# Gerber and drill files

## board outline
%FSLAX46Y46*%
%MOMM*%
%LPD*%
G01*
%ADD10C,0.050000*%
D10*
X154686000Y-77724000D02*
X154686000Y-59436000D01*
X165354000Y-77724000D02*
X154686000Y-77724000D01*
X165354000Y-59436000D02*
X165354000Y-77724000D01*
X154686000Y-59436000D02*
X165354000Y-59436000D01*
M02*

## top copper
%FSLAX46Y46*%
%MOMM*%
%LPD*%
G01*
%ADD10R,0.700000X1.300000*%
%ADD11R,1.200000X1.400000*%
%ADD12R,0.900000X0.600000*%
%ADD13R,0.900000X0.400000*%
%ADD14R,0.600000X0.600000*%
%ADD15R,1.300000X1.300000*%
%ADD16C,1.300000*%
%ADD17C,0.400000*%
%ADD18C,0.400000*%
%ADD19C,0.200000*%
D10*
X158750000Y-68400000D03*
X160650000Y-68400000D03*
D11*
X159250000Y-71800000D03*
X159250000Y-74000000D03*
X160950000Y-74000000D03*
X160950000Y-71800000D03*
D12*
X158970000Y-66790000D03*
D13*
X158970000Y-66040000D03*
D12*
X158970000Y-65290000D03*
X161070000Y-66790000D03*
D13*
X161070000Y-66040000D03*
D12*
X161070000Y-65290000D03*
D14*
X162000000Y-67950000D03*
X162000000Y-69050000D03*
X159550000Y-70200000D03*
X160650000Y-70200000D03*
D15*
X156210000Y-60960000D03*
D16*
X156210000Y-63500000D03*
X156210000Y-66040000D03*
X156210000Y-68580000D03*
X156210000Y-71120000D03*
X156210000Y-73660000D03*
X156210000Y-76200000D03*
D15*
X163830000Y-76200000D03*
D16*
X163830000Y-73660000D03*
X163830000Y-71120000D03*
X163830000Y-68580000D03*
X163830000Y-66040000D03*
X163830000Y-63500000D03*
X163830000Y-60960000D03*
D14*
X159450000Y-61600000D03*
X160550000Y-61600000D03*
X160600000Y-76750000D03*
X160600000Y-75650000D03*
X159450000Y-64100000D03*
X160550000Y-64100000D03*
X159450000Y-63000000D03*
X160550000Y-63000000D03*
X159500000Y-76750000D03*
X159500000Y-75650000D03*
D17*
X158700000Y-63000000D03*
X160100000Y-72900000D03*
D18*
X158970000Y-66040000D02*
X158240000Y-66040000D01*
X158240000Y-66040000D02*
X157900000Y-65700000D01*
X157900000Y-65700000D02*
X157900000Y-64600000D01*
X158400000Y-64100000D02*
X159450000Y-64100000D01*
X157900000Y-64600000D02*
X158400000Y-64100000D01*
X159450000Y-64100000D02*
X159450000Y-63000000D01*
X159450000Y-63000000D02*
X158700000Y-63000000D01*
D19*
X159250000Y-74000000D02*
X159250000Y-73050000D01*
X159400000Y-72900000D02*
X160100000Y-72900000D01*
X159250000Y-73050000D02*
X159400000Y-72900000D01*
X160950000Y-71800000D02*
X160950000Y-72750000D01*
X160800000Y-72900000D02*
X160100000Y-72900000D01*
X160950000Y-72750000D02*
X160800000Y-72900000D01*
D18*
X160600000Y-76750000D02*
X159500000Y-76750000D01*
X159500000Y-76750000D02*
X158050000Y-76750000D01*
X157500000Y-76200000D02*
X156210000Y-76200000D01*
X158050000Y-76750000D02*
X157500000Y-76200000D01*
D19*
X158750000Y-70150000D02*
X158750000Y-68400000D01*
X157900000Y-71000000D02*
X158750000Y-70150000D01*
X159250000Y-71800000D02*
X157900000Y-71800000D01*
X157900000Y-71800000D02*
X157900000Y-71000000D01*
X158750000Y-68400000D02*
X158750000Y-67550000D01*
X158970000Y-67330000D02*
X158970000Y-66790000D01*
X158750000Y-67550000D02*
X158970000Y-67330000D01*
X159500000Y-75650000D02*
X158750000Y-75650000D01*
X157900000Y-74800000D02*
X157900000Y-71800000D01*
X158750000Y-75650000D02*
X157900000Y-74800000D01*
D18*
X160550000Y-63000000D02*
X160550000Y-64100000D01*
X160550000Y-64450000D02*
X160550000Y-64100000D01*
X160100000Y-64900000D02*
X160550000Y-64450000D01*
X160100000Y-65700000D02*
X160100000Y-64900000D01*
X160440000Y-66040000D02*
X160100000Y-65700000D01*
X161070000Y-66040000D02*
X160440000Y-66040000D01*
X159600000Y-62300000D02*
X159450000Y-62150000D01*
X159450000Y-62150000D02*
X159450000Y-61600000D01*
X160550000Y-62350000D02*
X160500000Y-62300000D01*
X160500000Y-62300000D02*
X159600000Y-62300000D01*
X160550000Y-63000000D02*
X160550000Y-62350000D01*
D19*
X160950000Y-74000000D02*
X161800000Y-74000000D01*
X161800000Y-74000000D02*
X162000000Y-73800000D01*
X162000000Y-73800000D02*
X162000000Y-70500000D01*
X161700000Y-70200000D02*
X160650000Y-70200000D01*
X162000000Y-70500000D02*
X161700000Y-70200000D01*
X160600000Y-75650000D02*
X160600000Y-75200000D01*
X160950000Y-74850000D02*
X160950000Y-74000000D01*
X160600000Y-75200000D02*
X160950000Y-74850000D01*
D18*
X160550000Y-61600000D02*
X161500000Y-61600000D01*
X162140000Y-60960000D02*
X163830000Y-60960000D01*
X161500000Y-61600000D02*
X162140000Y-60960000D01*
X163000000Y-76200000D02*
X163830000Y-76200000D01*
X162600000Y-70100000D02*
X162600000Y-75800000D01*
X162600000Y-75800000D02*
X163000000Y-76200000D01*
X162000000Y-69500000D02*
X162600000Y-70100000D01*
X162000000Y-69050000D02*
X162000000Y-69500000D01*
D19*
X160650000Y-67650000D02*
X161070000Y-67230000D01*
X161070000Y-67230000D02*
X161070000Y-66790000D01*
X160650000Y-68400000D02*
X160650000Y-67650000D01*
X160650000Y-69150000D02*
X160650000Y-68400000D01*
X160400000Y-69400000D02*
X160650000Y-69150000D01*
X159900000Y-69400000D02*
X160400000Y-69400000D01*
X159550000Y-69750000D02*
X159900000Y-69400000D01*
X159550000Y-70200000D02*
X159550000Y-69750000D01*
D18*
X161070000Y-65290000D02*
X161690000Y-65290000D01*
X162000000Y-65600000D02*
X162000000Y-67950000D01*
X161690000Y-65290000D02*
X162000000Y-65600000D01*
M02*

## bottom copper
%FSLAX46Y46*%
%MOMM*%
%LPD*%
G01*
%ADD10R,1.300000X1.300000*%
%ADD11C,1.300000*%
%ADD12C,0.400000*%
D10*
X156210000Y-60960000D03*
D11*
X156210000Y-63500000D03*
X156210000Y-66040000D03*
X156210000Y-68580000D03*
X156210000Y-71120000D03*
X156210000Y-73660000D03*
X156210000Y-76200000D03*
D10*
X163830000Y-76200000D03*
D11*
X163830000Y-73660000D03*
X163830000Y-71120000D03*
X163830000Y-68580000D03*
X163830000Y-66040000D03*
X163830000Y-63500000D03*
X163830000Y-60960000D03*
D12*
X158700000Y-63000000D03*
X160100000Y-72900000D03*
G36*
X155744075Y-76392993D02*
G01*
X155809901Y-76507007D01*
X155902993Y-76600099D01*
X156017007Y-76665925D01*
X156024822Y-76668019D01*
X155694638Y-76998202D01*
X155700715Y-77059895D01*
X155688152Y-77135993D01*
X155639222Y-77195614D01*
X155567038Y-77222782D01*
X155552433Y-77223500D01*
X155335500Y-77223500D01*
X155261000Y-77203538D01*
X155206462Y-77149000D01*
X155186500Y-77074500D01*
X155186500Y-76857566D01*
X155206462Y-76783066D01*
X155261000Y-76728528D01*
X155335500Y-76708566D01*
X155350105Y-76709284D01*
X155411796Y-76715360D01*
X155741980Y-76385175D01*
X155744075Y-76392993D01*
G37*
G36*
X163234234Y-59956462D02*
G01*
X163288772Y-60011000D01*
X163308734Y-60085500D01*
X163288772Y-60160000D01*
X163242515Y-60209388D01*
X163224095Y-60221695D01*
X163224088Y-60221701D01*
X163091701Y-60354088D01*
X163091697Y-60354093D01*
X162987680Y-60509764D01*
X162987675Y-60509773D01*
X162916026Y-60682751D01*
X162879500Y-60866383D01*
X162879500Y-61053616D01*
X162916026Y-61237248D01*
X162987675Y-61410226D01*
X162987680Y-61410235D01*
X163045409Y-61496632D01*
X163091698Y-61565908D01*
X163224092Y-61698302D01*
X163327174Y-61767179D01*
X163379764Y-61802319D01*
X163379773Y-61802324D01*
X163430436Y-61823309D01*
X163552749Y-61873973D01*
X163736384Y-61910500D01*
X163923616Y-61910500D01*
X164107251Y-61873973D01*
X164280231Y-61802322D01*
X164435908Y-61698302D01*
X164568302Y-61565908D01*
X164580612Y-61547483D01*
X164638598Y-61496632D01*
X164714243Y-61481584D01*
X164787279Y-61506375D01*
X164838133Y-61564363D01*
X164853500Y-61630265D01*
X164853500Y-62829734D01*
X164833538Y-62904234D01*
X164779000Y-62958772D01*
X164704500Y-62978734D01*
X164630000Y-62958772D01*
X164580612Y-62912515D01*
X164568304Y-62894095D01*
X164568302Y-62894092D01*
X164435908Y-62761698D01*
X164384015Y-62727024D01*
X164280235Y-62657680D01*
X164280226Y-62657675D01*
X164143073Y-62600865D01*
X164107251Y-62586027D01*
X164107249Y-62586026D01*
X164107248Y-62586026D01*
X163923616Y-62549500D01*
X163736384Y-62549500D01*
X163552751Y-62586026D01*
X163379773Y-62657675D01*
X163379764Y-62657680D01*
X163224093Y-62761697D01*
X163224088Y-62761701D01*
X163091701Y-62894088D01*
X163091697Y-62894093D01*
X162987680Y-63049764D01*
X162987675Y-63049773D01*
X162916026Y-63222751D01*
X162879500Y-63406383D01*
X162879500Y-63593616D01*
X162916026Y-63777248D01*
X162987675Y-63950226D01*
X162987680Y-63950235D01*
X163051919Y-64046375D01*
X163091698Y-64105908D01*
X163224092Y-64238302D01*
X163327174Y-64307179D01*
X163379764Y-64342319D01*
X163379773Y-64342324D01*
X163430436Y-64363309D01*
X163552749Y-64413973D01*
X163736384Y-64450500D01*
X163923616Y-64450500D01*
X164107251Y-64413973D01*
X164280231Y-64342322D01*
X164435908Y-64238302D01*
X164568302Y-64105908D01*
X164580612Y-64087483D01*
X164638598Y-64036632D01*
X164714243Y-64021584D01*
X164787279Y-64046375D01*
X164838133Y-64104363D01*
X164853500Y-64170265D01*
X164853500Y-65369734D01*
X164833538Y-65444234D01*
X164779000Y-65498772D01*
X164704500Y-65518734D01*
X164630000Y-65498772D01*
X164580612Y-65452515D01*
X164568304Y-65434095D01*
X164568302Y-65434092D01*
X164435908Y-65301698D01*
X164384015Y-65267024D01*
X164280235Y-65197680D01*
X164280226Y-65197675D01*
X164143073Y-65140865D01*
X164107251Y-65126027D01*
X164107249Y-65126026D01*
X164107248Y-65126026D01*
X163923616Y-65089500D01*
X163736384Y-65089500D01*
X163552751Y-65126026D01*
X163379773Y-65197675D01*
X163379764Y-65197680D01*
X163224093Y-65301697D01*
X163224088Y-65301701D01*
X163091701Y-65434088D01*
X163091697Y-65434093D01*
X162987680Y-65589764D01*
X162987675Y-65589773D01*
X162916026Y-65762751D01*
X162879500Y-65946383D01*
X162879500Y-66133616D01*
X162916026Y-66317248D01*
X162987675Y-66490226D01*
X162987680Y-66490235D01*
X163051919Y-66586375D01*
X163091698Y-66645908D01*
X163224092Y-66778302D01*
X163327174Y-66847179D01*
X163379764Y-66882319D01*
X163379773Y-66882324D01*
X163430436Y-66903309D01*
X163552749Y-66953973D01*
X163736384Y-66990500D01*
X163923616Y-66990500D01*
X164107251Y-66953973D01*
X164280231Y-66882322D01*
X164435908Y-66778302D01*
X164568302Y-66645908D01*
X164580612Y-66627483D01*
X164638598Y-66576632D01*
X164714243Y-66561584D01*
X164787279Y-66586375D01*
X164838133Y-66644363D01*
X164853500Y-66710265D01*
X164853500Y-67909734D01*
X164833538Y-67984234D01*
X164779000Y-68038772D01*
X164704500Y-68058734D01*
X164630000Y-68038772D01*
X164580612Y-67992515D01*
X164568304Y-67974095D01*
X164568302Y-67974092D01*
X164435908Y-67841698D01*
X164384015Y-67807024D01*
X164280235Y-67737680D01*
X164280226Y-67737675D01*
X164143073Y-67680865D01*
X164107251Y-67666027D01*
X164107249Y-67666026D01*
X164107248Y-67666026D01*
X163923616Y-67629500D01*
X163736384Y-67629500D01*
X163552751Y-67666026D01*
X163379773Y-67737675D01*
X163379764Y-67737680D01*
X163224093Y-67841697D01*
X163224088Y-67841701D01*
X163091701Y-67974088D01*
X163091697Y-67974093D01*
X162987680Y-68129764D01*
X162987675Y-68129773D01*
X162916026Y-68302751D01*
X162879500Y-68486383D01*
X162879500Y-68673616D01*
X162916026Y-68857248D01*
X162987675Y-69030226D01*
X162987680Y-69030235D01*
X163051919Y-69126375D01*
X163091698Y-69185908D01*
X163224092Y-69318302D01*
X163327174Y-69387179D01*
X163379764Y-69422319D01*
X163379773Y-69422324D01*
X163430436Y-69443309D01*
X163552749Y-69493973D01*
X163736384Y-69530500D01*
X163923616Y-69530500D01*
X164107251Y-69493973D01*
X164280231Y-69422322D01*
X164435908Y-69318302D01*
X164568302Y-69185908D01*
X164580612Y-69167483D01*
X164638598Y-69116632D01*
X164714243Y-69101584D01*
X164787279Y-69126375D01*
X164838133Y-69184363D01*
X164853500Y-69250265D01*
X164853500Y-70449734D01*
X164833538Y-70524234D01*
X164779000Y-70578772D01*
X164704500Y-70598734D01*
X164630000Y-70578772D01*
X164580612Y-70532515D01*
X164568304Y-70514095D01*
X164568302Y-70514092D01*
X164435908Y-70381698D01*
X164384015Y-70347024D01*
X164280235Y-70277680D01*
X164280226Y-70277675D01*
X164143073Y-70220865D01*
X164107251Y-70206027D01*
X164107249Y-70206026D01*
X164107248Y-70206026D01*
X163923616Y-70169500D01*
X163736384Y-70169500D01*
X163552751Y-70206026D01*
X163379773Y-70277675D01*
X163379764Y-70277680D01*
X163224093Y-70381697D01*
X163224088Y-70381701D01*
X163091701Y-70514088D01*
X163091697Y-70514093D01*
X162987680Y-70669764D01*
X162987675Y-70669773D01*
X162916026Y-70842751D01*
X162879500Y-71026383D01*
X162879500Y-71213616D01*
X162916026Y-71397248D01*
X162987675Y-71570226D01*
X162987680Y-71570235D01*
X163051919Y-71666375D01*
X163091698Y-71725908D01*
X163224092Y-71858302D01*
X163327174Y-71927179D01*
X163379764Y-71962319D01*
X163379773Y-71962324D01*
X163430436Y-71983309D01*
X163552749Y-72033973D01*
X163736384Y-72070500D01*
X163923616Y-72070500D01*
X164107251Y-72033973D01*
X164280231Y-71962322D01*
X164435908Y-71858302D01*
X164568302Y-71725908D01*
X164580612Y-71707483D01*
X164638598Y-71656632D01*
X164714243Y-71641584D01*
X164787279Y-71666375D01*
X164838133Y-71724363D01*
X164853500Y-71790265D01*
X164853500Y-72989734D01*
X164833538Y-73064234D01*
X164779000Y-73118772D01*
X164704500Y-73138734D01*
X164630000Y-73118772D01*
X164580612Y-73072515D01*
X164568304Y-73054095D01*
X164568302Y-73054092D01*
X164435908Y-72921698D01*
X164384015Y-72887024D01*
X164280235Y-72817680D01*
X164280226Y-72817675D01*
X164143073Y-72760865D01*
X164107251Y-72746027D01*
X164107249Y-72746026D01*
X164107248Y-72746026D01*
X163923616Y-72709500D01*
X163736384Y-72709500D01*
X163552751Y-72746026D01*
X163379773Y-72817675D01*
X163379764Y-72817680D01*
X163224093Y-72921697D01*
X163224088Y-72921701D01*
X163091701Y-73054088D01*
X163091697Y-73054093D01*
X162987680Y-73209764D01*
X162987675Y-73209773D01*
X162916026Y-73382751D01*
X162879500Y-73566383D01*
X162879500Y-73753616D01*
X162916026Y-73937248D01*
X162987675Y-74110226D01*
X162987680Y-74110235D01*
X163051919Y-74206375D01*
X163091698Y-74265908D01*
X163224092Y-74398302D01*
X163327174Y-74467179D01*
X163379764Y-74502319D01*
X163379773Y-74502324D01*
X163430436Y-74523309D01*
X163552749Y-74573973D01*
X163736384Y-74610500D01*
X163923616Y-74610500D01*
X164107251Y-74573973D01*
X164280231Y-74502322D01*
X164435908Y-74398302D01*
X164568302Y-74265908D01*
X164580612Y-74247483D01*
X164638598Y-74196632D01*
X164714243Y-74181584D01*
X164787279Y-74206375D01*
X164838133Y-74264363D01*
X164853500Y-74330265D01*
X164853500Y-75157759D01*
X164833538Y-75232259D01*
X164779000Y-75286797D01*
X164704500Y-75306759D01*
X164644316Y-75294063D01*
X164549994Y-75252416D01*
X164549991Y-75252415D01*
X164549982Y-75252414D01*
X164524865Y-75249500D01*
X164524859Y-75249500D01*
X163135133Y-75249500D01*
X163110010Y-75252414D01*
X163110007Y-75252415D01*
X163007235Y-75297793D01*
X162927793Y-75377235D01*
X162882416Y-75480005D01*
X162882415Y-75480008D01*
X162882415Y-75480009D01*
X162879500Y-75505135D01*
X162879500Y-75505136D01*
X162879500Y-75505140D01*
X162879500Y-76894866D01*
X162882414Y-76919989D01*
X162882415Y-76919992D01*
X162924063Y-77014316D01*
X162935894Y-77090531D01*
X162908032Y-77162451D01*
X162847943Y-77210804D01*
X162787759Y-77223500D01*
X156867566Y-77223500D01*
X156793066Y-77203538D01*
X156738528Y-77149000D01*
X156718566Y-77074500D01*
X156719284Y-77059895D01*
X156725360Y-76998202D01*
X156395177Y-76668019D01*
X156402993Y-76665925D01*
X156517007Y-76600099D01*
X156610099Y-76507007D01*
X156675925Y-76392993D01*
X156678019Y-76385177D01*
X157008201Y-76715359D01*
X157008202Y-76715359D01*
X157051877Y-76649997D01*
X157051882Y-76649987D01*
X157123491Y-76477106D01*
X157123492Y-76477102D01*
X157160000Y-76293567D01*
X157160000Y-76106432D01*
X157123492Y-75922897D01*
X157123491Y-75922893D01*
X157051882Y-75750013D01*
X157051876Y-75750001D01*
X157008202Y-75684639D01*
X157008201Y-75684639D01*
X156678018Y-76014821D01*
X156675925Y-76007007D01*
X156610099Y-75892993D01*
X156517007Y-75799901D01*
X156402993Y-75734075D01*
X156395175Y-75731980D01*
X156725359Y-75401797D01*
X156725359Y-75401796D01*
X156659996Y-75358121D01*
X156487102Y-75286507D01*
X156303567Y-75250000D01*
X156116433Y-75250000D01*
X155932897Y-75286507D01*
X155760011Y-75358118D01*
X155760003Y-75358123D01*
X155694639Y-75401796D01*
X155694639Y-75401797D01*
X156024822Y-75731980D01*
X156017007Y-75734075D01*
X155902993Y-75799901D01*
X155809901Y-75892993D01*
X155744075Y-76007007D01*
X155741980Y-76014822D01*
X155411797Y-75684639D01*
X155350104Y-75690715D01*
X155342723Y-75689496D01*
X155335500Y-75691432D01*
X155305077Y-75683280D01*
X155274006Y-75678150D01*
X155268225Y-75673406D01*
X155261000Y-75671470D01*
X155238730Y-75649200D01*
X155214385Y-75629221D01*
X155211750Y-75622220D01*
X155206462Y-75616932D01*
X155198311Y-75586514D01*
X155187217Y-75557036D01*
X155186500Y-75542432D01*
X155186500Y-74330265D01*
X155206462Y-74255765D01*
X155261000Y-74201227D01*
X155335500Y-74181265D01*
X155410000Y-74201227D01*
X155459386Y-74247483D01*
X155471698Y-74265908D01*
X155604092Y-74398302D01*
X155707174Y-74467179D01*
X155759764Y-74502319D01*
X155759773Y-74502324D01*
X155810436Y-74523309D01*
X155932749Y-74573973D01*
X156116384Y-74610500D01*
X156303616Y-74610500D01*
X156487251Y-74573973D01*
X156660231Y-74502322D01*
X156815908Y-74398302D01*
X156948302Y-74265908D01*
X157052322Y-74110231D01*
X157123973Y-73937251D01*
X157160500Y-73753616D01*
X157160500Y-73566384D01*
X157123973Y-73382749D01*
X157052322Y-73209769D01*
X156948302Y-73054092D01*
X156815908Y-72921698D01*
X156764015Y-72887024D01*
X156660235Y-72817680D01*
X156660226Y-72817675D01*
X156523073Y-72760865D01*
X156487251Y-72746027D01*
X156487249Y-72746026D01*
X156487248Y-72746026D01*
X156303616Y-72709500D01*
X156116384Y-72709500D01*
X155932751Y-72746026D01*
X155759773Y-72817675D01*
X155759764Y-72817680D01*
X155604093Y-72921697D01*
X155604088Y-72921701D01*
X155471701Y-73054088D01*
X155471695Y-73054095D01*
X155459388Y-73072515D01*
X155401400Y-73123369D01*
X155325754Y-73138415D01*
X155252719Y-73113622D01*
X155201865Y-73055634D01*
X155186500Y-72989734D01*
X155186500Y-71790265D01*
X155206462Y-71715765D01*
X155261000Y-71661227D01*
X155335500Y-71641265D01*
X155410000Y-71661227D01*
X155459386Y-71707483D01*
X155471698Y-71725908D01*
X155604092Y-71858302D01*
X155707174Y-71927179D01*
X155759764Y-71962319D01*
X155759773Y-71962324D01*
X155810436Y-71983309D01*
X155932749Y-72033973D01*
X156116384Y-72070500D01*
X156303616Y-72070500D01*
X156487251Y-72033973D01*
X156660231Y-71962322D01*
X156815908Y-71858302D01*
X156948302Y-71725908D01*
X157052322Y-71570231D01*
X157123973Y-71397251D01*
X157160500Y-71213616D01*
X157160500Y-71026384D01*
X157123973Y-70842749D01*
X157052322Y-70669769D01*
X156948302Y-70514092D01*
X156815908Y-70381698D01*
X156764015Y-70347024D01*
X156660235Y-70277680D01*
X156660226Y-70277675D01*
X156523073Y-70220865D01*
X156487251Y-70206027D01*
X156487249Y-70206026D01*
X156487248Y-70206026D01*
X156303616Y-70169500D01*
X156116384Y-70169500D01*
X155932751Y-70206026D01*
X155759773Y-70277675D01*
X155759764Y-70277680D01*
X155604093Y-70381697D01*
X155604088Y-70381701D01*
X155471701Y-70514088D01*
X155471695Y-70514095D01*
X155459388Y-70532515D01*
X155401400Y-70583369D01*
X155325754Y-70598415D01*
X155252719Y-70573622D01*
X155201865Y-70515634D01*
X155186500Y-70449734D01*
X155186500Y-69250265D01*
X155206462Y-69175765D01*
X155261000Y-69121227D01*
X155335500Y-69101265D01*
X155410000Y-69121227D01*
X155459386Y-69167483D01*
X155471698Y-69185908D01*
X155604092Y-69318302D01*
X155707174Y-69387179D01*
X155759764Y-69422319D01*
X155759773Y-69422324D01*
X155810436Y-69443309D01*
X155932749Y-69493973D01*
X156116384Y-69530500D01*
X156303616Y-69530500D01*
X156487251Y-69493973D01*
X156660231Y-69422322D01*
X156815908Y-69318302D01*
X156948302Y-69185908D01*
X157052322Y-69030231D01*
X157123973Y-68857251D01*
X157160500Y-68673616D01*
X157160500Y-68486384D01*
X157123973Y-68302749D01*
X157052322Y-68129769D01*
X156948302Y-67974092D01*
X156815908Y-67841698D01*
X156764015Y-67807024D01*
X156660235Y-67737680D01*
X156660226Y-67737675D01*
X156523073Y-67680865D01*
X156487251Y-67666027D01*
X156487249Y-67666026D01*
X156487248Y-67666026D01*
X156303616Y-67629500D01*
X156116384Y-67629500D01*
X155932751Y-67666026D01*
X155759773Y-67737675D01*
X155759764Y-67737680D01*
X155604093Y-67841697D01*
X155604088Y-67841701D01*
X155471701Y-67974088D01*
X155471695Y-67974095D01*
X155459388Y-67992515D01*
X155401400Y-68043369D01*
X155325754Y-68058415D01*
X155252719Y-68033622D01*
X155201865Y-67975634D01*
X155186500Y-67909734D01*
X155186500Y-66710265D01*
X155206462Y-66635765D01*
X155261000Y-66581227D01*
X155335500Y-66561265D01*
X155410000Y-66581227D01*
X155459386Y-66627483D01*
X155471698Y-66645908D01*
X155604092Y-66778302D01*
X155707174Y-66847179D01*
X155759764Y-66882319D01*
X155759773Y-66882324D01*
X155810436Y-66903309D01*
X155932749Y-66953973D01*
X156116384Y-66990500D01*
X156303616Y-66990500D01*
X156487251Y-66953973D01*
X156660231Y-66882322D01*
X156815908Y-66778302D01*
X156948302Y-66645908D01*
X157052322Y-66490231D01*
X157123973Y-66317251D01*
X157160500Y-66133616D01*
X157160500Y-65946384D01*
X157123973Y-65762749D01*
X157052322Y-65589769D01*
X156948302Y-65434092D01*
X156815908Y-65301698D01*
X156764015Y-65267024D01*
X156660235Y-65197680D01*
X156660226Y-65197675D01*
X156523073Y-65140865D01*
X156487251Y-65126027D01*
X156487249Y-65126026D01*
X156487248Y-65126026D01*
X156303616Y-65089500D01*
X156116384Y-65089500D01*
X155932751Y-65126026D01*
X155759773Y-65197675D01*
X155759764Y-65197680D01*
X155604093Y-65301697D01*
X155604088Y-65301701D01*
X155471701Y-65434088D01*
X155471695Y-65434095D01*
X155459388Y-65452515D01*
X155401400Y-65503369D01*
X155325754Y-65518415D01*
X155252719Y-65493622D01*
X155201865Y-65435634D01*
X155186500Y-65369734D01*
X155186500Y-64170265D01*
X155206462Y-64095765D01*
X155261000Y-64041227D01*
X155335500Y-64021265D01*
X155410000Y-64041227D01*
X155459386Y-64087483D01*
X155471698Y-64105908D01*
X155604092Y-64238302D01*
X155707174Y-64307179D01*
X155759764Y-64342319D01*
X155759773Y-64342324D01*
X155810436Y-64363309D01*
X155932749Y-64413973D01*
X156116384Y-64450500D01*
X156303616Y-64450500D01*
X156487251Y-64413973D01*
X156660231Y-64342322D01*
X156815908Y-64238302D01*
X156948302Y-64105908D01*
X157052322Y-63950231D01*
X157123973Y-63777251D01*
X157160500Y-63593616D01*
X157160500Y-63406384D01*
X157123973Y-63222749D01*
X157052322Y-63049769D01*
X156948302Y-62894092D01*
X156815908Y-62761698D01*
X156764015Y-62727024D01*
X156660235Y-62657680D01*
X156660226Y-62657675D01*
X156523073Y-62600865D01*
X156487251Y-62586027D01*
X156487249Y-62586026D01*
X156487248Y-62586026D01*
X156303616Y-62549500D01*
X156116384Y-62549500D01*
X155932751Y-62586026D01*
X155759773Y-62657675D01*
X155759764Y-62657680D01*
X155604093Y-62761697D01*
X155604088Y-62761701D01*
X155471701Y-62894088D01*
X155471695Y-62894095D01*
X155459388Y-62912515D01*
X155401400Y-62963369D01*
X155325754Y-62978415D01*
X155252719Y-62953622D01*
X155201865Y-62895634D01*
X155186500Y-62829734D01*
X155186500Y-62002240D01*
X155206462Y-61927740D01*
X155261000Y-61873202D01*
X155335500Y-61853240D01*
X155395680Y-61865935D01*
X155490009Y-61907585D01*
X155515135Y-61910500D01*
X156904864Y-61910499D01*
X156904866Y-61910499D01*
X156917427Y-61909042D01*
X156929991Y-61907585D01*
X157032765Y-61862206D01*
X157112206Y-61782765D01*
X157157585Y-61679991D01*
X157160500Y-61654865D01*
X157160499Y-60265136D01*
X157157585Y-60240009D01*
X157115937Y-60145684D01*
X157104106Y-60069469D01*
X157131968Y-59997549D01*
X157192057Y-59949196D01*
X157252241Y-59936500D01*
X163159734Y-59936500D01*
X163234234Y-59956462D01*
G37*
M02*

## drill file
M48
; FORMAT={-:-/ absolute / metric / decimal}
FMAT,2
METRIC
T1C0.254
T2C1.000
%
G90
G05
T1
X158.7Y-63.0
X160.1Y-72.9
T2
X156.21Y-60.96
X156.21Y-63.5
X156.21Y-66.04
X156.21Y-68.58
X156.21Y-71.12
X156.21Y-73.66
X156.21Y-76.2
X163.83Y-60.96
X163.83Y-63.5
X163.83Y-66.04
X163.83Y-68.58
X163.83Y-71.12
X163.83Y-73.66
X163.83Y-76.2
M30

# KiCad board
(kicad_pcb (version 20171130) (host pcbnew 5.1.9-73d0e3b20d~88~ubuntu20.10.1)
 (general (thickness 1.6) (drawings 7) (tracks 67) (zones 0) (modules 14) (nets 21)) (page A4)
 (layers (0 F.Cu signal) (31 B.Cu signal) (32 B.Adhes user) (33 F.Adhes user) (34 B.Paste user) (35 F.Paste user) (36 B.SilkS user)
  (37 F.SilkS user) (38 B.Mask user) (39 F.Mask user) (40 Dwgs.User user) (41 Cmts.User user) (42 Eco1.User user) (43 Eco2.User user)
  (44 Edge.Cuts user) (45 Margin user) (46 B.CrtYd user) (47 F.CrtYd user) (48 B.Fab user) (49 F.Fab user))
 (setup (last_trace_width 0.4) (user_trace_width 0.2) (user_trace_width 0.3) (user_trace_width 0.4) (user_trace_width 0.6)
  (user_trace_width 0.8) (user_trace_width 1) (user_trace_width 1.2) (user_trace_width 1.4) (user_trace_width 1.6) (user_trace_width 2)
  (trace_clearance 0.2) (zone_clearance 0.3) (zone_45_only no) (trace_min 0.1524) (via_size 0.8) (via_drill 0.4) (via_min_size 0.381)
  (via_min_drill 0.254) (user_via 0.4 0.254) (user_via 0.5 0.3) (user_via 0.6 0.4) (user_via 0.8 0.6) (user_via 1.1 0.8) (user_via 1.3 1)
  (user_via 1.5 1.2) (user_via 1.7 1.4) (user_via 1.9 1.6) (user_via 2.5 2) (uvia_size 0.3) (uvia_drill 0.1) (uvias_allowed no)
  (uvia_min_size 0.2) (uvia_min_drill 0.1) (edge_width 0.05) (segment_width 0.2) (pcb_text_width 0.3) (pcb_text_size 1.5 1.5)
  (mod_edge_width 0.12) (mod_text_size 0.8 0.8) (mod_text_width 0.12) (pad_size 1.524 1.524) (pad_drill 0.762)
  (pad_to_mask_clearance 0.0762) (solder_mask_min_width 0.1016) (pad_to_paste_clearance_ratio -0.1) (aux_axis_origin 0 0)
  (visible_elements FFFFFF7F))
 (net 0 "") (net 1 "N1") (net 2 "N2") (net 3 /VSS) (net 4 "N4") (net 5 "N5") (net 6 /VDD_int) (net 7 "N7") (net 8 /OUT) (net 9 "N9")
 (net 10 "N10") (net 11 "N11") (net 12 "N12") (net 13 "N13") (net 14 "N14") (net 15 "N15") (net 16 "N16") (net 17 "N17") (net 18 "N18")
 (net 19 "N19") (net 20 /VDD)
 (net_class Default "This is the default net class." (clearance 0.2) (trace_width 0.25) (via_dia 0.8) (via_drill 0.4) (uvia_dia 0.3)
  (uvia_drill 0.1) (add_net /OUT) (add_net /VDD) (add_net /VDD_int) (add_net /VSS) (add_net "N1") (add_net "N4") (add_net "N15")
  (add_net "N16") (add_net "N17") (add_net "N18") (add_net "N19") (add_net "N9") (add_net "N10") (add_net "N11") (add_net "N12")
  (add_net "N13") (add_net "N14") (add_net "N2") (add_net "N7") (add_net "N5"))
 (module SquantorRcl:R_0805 (layer F.Cu) (at 159.7 68.4 180)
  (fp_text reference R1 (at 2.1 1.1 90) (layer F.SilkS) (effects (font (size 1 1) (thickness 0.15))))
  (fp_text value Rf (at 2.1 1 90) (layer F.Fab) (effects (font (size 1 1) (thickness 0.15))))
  (pad 2 smd rect (at 0.95 0 180) (size 0.7 1.3) (layers F.Cu F.Paste F.Mask) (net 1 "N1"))
  (pad 1 smd rect (at -0.95 0 180) (size 0.7 1.3) (layers F.Cu F.Paste F.Mask) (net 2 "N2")))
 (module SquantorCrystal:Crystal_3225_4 (layer F.Cu) (at 160.1 72.9 270)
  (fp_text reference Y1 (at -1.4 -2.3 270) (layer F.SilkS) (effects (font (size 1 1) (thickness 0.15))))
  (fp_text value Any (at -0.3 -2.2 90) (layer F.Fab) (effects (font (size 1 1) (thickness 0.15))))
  (pad 1 smd rect (at -1.1 0.85 270) (size 1.4 1.2) (layers F.Cu F.Paste F.Mask) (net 1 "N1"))
  (pad 2 smd rect (at 1.1 0.85 270) (size 1.4 1.2) (layers F.Cu F.Paste F.Mask) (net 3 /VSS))
  (pad 3 smd rect (at 1.1 -0.85 270) (size 1.4 1.2) (layers F.Cu F.Paste F.Mask) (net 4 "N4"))
  (pad 4 smd rect (at -1.1 -0.85 270) (size 1.4 1.2) (layers F.Cu F.Paste F.Mask) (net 3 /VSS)))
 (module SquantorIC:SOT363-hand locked (layer F.Cu) (at 160.02 66.04 270)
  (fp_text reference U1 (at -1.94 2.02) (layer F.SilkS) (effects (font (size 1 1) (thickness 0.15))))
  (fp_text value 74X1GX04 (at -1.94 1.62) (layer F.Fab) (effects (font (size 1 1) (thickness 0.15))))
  (pad 3 smd rect (at 0.75 1.05 270) (size 0.6 0.9) (layers F.Cu F.Paste F.Mask) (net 1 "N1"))
  (pad 2 smd rect (at 0 1.05 270) (size 0.4 0.9) (layers F.Cu F.Paste F.Mask) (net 3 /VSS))
  (pad 1 smd rect (at -0.75 1.05 270) (size 0.6 0.9) (layers F.Cu F.Paste F.Mask) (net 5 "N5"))
  (pad 4 smd rect (at 0.75 -1.05 270) (size 0.6 0.9) (layers F.Cu F.Paste F.Mask) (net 2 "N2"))
  (pad 5 smd rect (at 0 -1.05 270) (size 0.4 0.9) (layers F.Cu F.Paste F.Mask) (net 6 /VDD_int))
  (pad 6 smd rect (at -0.75 -1.05 270) (size 0.6 0.9) (layers F.Cu F.Paste F.Mask) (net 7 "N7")))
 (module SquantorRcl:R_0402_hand (layer F.Cu) (at 162 68.5 90)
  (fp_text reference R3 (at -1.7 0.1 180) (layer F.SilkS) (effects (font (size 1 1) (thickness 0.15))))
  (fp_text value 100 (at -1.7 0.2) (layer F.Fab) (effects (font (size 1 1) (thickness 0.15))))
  (pad 2 smd rect (at 0.55 0 90) (size 0.6 0.6) (layers F.Cu F.Paste F.Mask) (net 7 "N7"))
  (pad 1 smd rect (at -0.55 0 90) (size 0.6 0.6) (layers F.Cu F.Paste F.Mask) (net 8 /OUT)))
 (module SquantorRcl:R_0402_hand (layer F.Cu) (at 160.1 70.2 180)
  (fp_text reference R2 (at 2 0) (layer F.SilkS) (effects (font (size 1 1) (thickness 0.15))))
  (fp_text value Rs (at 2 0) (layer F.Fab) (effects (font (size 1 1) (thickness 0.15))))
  (pad 2 smd rect (at 0.55 0 180) (size 0.6 0.6) (layers F.Cu F.Paste F.Mask) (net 2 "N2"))
  (pad 1 smd rect (at -0.55 0 180) (size 0.6 0.6) (layers F.Cu F.Paste F.Mask) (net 4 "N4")))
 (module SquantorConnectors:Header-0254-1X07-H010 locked (layer B.Cu) (at 156.21 68.58 270)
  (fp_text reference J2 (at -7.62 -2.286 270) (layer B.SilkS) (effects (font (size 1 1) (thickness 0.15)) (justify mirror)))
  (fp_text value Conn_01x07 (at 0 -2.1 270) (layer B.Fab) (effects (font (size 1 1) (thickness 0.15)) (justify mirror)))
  (pad 1 thru_hole rect (at -7.62 0 90) (size 1.3 1.3) (drill 1) (layers *.Cu *.Mask) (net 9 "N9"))
  (pad 2 thru_hole circle (at -5.08 0 90) (size 1.3 1.3) (drill 1) (layers *.Cu *.Mask) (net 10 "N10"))
  (pad 3 thru_hole circle (at -2.54 0 90) (size 1.3 1.3) (drill 1) (layers *.Cu *.Mask) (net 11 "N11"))
  (pad 4 thru_hole circle (at 0 0 90) (size 1.3 1.3) (drill 1) (layers *.Cu *.Mask) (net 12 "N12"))
  (pad 5 thru_hole circle (at 2.54 0 90) (size 1.3 1.3) (drill 1) (layers *.Cu *.Mask) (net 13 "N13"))
  (pad 6 thru_hole circle (at 5.08 0 90) (size 1.3 1.3) (drill 1) (layers *.Cu *.Mask) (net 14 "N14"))
  (pad 7 thru_hole circle (at 7.62 0 90) (size 1.3 1.3) (drill 1) (layers *.Cu *.Mask) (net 3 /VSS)))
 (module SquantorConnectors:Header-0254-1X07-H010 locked (layer B.Cu) (at 163.83 68.58 90)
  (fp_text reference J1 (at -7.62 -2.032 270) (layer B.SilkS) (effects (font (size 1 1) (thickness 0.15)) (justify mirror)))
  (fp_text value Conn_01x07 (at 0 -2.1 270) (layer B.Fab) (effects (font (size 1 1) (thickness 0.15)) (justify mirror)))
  (pad 1 thru_hole rect (at -7.62 0 270) (size 1.3 1.3) (drill 1) (layers *.Cu *.Mask) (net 8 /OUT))
  (pad 2 thru_hole circle (at -5.08 0 270) (size 1.3 1.3) (drill 1) (layers *.Cu *.Mask) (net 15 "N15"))
  (pad 3 thru_hole circle (at -2.54 0 270) (size 1.3 1.3) (drill 1) (layers *.Cu *.Mask) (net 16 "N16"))
  (pad 4 thru_hole circle (at 0 0 270) (size 1.3 1.3) (drill 1) (layers *.Cu *.Mask) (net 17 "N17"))
  (pad 5 thru_hole circle (at 2.54 0 270) (size 1.3 1.3) (drill 1) (layers *.Cu *.Mask) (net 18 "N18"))
  (pad 6 thru_hole circle (at 5.08 0 270) (size 1.3 1.3) (drill 1) (layers *.Cu *.Mask) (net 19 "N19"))
  (pad 7 thru_hole circle (at 7.62 0 270) (size 1.3 1.3) (drill 1) (layers *.Cu *.Mask) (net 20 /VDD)))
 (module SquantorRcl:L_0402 (layer F.Cu) (at 160 61.6 180)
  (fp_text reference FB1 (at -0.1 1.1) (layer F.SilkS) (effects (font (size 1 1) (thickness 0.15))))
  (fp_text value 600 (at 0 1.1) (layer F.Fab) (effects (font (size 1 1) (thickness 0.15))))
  (pad 2 smd rect (at 0.55 0 180) (size 0.6 0.6) (layers F.Cu F.Paste F.Mask) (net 6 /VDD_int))
  (pad 1 smd rect (at -0.55 0 180) (size 0.6 0.6) (layers F.Cu F.Paste F.Mask) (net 20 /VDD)))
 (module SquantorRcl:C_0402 (layer F.Cu) (at 160.6 76.2 270)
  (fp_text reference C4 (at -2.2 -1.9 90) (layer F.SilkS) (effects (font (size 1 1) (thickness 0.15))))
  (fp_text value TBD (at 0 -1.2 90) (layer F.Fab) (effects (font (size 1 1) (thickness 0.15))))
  (pad 2 smd rect (at 0.55 0 270) (size 0.6 0.6) (layers F.Cu F.Paste F.Mask) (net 3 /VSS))
  (pad 1 smd rect (at -0.55 0 270) (size 0.6 0.6) (layers F.Cu F.Paste F.Mask) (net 4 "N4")))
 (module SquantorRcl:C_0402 (layer F.Cu) (at 160 64.1 180)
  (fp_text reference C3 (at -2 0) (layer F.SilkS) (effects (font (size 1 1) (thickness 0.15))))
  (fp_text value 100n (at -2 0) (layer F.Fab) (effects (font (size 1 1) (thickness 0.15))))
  (pad 2 smd rect (at 0.55 0 180) (size 0.6 0.6) (layers F.Cu F.Paste F.Mask) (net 3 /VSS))
  (pad 1 smd rect (at -0.55 0 180) (size 0.6 0.6) (layers F.Cu F.Paste F.Mask) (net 6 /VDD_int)))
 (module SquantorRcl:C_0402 (layer F.Cu) (at 160 63 180)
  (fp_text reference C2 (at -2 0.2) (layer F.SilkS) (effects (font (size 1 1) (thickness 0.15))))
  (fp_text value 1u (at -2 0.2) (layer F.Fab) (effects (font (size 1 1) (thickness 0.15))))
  (pad 2 smd rect (at 0.55 0 180) (size 0.6 0.6) (layers F.Cu F.Paste F.Mask) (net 3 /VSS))
  (pad 1 smd rect (at -0.55 0 180) (size 0.6 0.6) (layers F.Cu F.Paste F.Mask) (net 6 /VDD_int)))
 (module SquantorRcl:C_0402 (layer F.Cu) (at 159.5 76.2 270)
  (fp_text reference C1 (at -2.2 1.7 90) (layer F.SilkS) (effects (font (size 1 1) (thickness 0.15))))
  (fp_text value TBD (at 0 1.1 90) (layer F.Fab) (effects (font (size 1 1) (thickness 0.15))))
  (pad 2 smd rect (at 0.55 0 270) (size 0.6 0.6) (layers F.Cu F.Paste F.Mask) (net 3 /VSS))
  (pad 1 smd rect (at -0.55 0 270) (size 0.6 0.6) (layers F.Cu F.Paste F.Mask) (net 1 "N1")))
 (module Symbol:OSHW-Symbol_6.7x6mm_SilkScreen (layer B.Cu) (at 160.02 69.596 180)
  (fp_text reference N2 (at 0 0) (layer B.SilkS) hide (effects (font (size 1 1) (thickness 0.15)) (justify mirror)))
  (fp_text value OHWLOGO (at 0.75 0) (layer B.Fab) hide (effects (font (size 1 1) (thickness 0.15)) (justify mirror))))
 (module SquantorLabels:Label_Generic (layer B.Cu) (at 159.385 74.93)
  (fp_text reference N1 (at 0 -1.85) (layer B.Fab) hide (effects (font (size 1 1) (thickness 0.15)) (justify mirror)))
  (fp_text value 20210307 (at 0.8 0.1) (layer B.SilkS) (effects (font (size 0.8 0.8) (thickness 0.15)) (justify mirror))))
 (gr_line (start 154.686 77.724) (end 154.686 59.436) (layer Edge.Cuts) (width 0.05))
 (gr_line (start 165.354 77.724) (end 154.686 77.724) (layer Edge.Cuts) (width 0.05))
 (gr_line (start 165.354 59.436) (end 165.354 77.724) (layer Edge.Cuts) (width 0.05))
 (gr_line (start 154.686 59.436) (end 165.354 59.436) (layer Edge.Cuts) (width 0.05))
 (segment (start 158.97 66.04) (end 158.24 66.04) (width 0.4) (layer F.Cu) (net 3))
 (segment (start 158.24 66.04) (end 157.9 65.7) (width 0.4) (layer F.Cu) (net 3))
 (segment (start 157.9 65.7) (end 157.9 64.6) (width 0.4) (layer F.Cu) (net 3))
 (segment (start 158.4 64.1) (end 159.45 64.1) (width 0.4) (layer F.Cu) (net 3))
 (segment (start 157.9 64.6) (end 158.4 64.1) (width 0.4) (layer F.Cu) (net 3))
 (segment (start 159.45 64.1) (end 159.45 63) (width 0.4) (layer F.Cu) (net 3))
 (via (at 158.7 63) (size 0.4) (drill 0.254) (layers F.Cu B.Cu) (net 3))
 (segment (start 159.45 63) (end 158.7 63) (width 0.4) (layer F.Cu) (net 3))
 (segment (start 159.25 74) (end 159.25 73.05) (width 0.2) (layer F.Cu) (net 3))
 (via (at 160.1 72.9) (size 0.4) (drill 0.254) (layers F.Cu B.Cu) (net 3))
 (segment (start 159.4 72.9) (end 160.1 72.9) (width 0.2) (layer F.Cu) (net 3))
 (segment (start 159.25 73.05) (end 159.4 72.9) (width 0.2) (layer F.Cu) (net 3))
 (segment (start 160.95 71.8) (end 160.95 72.75) (width 0.2) (layer F.Cu) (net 3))
 (segment (start 160.8 72.9) (end 160.1 72.9) (width 0.2) (layer F.Cu) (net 3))
 (segment (start 160.95 72.75) (end 160.8 72.9) (width 0.2) (layer F.Cu) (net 3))
 (segment (start 160.6 76.75) (end 159.5 76.75) (width 0.4) (layer F.Cu) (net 3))
 (segment (start 159.5 76.75) (end 158.05 76.75) (width 0.4) (layer F.Cu) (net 3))
 (segment (start 157.5 76.2) (end 156.21 76.2) (width 0.4) (layer F.Cu) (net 3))
 (segment (start 158.05 76.75) (end 157.5 76.2) (width 0.4) (layer F.Cu) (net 3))
 (segment (start 158.75 70.15) (end 158.75 68.4) (width 0.2) (layer F.Cu) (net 1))
 (segment (start 157.9 71) (end 158.75 70.15) (width 0.2) (layer F.Cu) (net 1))
 (segment (start 159.25 71.8) (end 157.9 71.8) (width 0.2) (layer F.Cu) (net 1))
 (segment (start 157.9 71.8) (end 157.9 71) (width 0.2) (layer F.Cu) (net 1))
 (segment (start 158.75 68.4) (end 158.75 67.55) (width 0.2) (layer F.Cu) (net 1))
 (segment (start 158.97 67.33) (end 158.97 66.79) (width 0.2) (layer F.Cu) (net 1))
 (segment (start 158.75 67.55) (end 158.97 67.33) (width 0.2) (layer F.Cu) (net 1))
 (segment (start 159.5 75.65) (end 158.75 75.65) (width 0.2) (layer F.Cu) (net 1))
 (segment (start 157.9 74.8) (end 157.9 71.8) (width 0.2) (layer F.Cu) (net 1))
 (segment (start 158.75 75.65) (end 157.9 74.8) (width 0.2) (layer F.Cu) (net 1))
 (segment (start 160.55 63) (end 160.55 64.1) (width 0.4) (layer F.Cu) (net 6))
 (segment (start 160.55 64.45) (end 160.55 64.1) (width 0.4) (layer F.Cu) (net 6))
 (segment (start 160.1 64.9) (end 160.55 64.45) (width 0.4) (layer F.Cu) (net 6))
 (segment (start 160.1 65.7) (end 160.1 64.9) (width 0.4) (layer F.Cu) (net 6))
 (segment (start 160.44 66.04) (end 160.1 65.7) (width 0.4) (layer F.Cu) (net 6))
 (segment (start 161.07 66.04) (end 160.44 66.04) (width 0.4) (layer F.Cu) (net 6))
 (segment (start 159.6 62.3) (end 159.45 62.15) (width 0.4) (layer F.Cu) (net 6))
 (segment (start 159.45 62.15) (end 159.45 61.6) (width 0.4) (layer F.Cu) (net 6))
 (segment (start 160.55 62.35) (end 160.5 62.3) (width 0.4) (layer F.Cu) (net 6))
 (segment (start 160.5 62.3) (end 159.6 62.3) (width 0.4) (layer F.Cu) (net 6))
 (segment (start 160.55 63) (end 160.55 62.35) (width 0.4) (layer F.Cu) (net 6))
 (segment (start 160.95 74) (end 161.8 74) (width 0.2) (layer F.Cu) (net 4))
 (segment (start 161.8 74) (end 162 73.8) (width 0.2) (layer F.Cu) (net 4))
 (segment (start 162 73.8) (end 162 70.5) (width 0.2) (layer F.Cu) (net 4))
 (segment (start 161.7 70.2) (end 160.65 70.2) (width 0.2) (layer F.Cu) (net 4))
 (segment (start 162 70.5) (end 161.7 70.2) (width 0.2) (layer F.Cu) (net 4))
 (segment (start 160.6 75.65) (end 160.6 75.2) (width 0.2) (layer F.Cu) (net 4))
 (segment (start 160.95 74.85) (end 160.95 74) (width 0.2) (layer F.Cu) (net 4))
 (segment (start 160.6 75.2) (end 160.95 74.85) (width 0.2) (layer F.Cu) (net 4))
 (segment (start 160.55 61.6) (end 161.5 61.6) (width 0.4) (layer F.Cu) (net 20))
 (segment (start 162.14 60.96) (end 163.83 60.96) (width 0.4) (layer F.Cu) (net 20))
 (segment (start 161.5 61.6) (end 162.14 60.96) (width 0.4) (layer F.Cu) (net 20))
 (segment (start 163 76.2) (end 163.83 76.2) (width 0.4) (layer F.Cu) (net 8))
 (segment (start 162.6 70.1) (end 162.6 75.8) (width 0.4) (layer F.Cu) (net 8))
 (segment (start 162.6 75.8) (end 163 76.2) (width 0.4) (layer F.Cu) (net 8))
 (segment (start 162 69.5) (end 162.6 70.1) (width 0.4) (layer F.Cu) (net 8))
 (segment (start 162 69.05) (end 162 69.5) (width 0.4) (layer F.Cu) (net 8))
 (segment (start 160.65 67.65) (end 161.07 67.23) (width 0.2) (layer F.Cu) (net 2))
 (segment (start 161.07 67.23) (end 161.07 66.79) (width 0.2) (layer F.Cu) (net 2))
 (segment (start 160.65 68.4) (end 160.65 67.65) (width 0.2) (layer F.Cu) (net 2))
 (segment (start 160.65 69.15) (end 160.65 68.4) (width 0.2) (layer F.Cu) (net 2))
 (segment (start 160.4 69.4) (end 160.65 69.15) (width 0.2) (layer F.Cu) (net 2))
 (segment (start 159.9 69.4) (end 160.4 69.4) (width 0.2) (layer F.Cu) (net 2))
 (segment (start 159.55 69.75) (end 159.9 69.4) (width 0.2) (layer F.Cu) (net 2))
 (segment (start 159.55 70.2) (end 159.55 69.75) (width 0.2) (layer F.Cu) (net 2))
 (segment (start 161.07 65.29) (end 161.69 65.29) (width 0.4) (layer F.Cu) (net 7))
 (segment (start 162 65.6) (end 162 67.95) (width 0.4) (layer F.Cu) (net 7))
 (segment (start 161.69 65.29) (end 162 65.6) (width 0.4) (layer F.Cu) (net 7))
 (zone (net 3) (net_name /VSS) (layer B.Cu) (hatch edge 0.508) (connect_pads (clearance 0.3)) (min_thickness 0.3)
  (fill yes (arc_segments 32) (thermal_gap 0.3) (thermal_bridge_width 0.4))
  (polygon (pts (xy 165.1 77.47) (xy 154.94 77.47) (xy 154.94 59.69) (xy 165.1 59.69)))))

